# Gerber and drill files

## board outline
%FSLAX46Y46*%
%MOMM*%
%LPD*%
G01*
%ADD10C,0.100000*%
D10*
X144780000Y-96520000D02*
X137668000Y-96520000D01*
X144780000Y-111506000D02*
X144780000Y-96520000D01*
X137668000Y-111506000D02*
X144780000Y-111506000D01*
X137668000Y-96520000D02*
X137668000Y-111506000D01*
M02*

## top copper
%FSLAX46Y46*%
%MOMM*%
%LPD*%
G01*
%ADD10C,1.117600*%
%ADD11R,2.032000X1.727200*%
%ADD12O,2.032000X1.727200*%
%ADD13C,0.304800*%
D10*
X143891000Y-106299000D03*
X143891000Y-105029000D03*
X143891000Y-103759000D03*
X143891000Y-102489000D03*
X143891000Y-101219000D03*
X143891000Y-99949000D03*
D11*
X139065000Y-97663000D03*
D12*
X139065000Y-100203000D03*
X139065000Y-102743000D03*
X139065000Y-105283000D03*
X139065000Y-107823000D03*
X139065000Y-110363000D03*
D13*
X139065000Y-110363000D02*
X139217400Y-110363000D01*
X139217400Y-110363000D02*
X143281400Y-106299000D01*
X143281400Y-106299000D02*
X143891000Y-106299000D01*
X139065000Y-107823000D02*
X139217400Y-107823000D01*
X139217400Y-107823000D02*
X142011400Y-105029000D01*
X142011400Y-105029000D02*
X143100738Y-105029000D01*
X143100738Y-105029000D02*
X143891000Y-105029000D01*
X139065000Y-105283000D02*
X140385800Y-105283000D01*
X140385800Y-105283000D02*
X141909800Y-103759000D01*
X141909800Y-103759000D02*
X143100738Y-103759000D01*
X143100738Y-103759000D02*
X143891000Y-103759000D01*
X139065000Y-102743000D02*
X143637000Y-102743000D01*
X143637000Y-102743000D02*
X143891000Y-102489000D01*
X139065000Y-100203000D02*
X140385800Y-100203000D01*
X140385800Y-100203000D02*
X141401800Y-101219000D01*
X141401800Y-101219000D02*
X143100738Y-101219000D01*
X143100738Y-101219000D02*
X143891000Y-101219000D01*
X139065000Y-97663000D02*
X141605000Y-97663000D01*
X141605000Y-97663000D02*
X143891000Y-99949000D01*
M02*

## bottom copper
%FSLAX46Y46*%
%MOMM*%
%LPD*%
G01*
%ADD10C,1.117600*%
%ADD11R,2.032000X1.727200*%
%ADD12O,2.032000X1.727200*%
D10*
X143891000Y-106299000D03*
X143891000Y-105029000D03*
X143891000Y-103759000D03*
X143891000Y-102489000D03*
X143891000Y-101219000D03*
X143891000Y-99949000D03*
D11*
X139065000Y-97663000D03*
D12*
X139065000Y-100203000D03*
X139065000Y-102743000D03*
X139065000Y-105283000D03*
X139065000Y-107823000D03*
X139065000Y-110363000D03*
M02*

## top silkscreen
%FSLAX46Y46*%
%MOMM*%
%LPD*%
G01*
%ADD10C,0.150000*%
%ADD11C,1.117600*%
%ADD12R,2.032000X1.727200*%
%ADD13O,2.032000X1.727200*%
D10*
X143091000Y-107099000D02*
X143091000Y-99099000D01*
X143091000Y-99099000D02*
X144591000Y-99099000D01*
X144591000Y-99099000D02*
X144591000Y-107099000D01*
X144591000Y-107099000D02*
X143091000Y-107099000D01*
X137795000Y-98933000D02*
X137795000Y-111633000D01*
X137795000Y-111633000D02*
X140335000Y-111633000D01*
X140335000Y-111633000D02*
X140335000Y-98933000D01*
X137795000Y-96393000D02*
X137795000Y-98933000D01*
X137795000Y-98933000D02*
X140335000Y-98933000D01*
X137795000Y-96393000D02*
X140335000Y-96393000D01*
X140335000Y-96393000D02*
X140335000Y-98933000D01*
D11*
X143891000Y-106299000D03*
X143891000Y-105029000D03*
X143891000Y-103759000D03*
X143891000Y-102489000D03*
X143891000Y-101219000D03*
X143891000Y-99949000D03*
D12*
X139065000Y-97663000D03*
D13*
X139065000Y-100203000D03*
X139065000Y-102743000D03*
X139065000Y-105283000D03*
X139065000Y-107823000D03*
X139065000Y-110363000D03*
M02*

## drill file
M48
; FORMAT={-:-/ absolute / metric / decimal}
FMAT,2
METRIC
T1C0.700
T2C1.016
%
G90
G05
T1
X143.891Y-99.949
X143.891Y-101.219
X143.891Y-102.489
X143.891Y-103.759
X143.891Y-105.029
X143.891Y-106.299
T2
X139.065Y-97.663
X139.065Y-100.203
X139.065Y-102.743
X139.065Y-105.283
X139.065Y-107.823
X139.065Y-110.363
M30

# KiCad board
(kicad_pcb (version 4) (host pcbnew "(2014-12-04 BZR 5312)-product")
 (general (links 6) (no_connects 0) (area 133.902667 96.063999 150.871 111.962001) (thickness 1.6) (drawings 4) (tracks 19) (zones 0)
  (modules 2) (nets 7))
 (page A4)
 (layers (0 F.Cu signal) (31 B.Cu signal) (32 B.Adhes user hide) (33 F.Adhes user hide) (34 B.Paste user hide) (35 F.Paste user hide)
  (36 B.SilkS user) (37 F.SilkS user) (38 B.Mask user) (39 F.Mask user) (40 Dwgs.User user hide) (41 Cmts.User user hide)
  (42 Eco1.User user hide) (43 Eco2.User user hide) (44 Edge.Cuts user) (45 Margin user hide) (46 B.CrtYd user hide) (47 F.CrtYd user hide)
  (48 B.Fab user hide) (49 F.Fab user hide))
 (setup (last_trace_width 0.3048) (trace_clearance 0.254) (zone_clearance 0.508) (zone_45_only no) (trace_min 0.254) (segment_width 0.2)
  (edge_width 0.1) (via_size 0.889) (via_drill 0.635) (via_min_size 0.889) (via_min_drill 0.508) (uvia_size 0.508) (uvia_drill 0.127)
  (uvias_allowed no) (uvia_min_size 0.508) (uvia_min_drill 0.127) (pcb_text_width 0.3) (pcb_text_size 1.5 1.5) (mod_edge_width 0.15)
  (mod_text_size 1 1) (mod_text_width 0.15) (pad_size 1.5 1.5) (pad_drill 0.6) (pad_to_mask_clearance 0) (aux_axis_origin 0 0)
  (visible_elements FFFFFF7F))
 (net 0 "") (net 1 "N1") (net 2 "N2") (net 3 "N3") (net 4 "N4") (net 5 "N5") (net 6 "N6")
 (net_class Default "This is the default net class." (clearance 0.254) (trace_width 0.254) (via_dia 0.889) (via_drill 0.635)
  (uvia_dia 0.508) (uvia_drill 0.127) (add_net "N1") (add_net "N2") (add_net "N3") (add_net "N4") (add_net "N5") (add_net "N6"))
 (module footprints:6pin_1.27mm (layer F.Cu) (at 143.891 106.299 90) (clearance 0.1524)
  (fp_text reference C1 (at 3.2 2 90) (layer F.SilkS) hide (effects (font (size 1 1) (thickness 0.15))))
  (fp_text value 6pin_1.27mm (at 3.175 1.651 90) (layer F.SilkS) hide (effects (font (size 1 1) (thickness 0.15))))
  (fp_line (start -0.8 -0.8) (end 7.2 -0.8) (layer F.SilkS) (width 0.15))
  (fp_line (start 7.2 -0.8) (end 7.2 0.7) (layer F.SilkS) (width 0.15))
  (fp_line (start 7.2 0.7) (end -0.8 0.7) (layer F.SilkS) (width 0.15))
  (fp_line (start -0.8 0.7) (end -0.8 -0.8) (layer F.SilkS) (width 0.15))
  (pad 1 thru_hole circle (at 0 0 90) (size 1.1176 1.1176) (drill 0.7) (layers *.Cu *.Mask F.SilkS) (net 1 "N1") (clearance 0.1524))
  (pad 2 thru_hole circle (at 1.27 0 90) (size 1.1176 1.1176) (drill 0.7) (layers *.Cu *.Mask F.SilkS) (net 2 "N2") (clearance 0.1524))
  (pad 3 thru_hole circle (at 2.54 0 90) (size 1.1176 1.1176) (drill 0.7) (layers *.Cu *.Mask F.SilkS) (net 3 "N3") (clearance 0.1524))
  (pad 4 thru_hole circle (at 3.81 0 90) (size 1.1176 1.1176) (drill 0.7) (layers *.Cu *.Mask F.SilkS) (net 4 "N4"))
  (pad 5 thru_hole circle (at 5.08 0 90) (size 1.1176 1.1176) (drill 0.7) (layers *.Cu *.Mask F.SilkS) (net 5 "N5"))
  (pad 6 thru_hole circle (at 6.35 0 90) (size 1.1176 1.1176) (drill 0.7) (layers *.Cu *.Mask F.SilkS) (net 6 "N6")))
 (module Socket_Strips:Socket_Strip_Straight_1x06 (layer F.Cu) (at 139.065 104.013 90)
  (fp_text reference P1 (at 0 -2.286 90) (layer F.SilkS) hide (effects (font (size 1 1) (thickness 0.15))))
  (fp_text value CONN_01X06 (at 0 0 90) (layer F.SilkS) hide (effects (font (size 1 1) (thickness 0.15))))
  (fp_line (start 5.08 -1.27) (end -7.62 -1.27) (layer F.SilkS) (width 0.15))
  (fp_line (start -7.62 -1.27) (end -7.62 1.27) (layer F.SilkS) (width 0.15))
  (fp_line (start -7.62 1.27) (end 5.08 1.27) (layer F.SilkS) (width 0.15))
  (fp_line (start 7.62 -1.27) (end 5.08 -1.27) (layer F.SilkS) (width 0.15))
  (fp_line (start 5.08 -1.27) (end 5.08 1.27) (layer F.SilkS) (width 0.15))
  (fp_line (start 7.62 -1.27) (end 7.62 1.27) (layer F.SilkS) (width 0.15))
  (fp_line (start 7.62 1.27) (end 5.08 1.27) (layer F.SilkS) (width 0.15))
  (pad 1 thru_hole rect (at 6.35 0 270) (size 1.7272 2.032) (drill 1.016) (layers *.Cu *.Mask F.SilkS) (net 6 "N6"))
  (pad 2 thru_hole oval (at 3.81 0 270) (size 1.7272 2.032) (drill 1.016) (layers *.Cu *.Mask F.SilkS) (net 5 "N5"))
  (pad 3 thru_hole oval (at 1.27 0 270) (size 1.7272 2.032) (drill 1.016) (layers *.Cu *.Mask F.SilkS) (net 4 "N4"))
  (pad 4 thru_hole oval (at -1.27 0 270) (size 1.7272 2.032) (drill 1.016) (layers *.Cu *.Mask F.SilkS) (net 3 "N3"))
  (pad 5 thru_hole oval (at -3.81 0 270) (size 1.7272 2.032) (drill 1.016) (layers *.Cu *.Mask F.SilkS) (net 2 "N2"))
  (pad 6 thru_hole oval (at -6.35 0 270) (size 1.7272 2.032) (drill 1.016) (layers *.Cu *.Mask F.SilkS) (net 1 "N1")))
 (gr_line (start 144.78 96.52) (end 137.668 96.52) (angle 90) (layer Edge.Cuts) (width 0.1))
 (gr_line (start 144.78 111.506) (end 144.78 96.52) (angle 90) (layer Edge.Cuts) (width 0.1))
 (gr_line (start 137.668 111.506) (end 144.78 111.506) (angle 90) (layer Edge.Cuts) (width 0.1))
 (gr_line (start 137.668 96.52) (end 137.668 111.506) (angle 90) (layer Edge.Cuts) (width 0.1))
 (segment (start 139.065 110.363) (end 139.2174 110.363) (width 0.3048) (layer F.Cu) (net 1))
 (segment (start 139.2174 110.363) (end 143.2814 106.299) (width 0.3048) (layer F.Cu) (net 1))
 (segment (start 143.2814 106.299) (end 143.891 106.299) (width 0.3048) (layer F.Cu) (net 1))
 (segment (start 139.065 107.823) (end 139.2174 107.823) (width 0.3048) (layer F.Cu) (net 2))
 (segment (start 139.2174 107.823) (end 142.0114 105.029) (width 0.3048) (layer F.Cu) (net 2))
 (segment (start 142.0114 105.029) (end 143.100738 105.029) (width 0.3048) (layer F.Cu) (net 2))
 (segment (start 143.100738 105.029) (end 143.891 105.029) (width 0.3048) (layer F.Cu) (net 2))
 (segment (start 139.065 105.283) (end 140.3858 105.283) (width 0.3048) (layer F.Cu) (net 3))
 (segment (start 140.3858 105.283) (end 141.9098 103.759) (width 0.3048) (layer F.Cu) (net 3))
 (segment (start 141.9098 103.759) (end 143.100738 103.759) (width 0.3048) (layer F.Cu) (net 3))
 (segment (start 143.100738 103.759) (end 143.891 103.759) (width 0.3048) (layer F.Cu) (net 3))
 (segment (start 139.065 102.743) (end 143.637 102.743) (width 0.3048) (layer F.Cu) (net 4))
 (segment (start 143.637 102.743) (end 143.891 102.489) (width 0.3048) (layer F.Cu) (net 4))
 (segment (start 139.065 100.203) (end 140.3858 100.203) (width 0.3048) (layer F.Cu) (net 5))
 (segment (start 140.3858 100.203) (end 141.4018 101.219) (width 0.3048) (layer F.Cu) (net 5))
 (segment (start 141.4018 101.219) (end 143.100738 101.219) (width 0.3048) (layer F.Cu) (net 5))
 (segment (start 143.100738 101.219) (end 143.891 101.219) (width 0.3048) (layer F.Cu) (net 5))
 (segment (start 139.065 97.663) (end 141.605 97.663) (width 0.3048) (layer F.Cu) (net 6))
 (segment (start 141.605 97.663) (end 143.891 99.949) (width 0.3048) (layer F.Cu) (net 6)))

